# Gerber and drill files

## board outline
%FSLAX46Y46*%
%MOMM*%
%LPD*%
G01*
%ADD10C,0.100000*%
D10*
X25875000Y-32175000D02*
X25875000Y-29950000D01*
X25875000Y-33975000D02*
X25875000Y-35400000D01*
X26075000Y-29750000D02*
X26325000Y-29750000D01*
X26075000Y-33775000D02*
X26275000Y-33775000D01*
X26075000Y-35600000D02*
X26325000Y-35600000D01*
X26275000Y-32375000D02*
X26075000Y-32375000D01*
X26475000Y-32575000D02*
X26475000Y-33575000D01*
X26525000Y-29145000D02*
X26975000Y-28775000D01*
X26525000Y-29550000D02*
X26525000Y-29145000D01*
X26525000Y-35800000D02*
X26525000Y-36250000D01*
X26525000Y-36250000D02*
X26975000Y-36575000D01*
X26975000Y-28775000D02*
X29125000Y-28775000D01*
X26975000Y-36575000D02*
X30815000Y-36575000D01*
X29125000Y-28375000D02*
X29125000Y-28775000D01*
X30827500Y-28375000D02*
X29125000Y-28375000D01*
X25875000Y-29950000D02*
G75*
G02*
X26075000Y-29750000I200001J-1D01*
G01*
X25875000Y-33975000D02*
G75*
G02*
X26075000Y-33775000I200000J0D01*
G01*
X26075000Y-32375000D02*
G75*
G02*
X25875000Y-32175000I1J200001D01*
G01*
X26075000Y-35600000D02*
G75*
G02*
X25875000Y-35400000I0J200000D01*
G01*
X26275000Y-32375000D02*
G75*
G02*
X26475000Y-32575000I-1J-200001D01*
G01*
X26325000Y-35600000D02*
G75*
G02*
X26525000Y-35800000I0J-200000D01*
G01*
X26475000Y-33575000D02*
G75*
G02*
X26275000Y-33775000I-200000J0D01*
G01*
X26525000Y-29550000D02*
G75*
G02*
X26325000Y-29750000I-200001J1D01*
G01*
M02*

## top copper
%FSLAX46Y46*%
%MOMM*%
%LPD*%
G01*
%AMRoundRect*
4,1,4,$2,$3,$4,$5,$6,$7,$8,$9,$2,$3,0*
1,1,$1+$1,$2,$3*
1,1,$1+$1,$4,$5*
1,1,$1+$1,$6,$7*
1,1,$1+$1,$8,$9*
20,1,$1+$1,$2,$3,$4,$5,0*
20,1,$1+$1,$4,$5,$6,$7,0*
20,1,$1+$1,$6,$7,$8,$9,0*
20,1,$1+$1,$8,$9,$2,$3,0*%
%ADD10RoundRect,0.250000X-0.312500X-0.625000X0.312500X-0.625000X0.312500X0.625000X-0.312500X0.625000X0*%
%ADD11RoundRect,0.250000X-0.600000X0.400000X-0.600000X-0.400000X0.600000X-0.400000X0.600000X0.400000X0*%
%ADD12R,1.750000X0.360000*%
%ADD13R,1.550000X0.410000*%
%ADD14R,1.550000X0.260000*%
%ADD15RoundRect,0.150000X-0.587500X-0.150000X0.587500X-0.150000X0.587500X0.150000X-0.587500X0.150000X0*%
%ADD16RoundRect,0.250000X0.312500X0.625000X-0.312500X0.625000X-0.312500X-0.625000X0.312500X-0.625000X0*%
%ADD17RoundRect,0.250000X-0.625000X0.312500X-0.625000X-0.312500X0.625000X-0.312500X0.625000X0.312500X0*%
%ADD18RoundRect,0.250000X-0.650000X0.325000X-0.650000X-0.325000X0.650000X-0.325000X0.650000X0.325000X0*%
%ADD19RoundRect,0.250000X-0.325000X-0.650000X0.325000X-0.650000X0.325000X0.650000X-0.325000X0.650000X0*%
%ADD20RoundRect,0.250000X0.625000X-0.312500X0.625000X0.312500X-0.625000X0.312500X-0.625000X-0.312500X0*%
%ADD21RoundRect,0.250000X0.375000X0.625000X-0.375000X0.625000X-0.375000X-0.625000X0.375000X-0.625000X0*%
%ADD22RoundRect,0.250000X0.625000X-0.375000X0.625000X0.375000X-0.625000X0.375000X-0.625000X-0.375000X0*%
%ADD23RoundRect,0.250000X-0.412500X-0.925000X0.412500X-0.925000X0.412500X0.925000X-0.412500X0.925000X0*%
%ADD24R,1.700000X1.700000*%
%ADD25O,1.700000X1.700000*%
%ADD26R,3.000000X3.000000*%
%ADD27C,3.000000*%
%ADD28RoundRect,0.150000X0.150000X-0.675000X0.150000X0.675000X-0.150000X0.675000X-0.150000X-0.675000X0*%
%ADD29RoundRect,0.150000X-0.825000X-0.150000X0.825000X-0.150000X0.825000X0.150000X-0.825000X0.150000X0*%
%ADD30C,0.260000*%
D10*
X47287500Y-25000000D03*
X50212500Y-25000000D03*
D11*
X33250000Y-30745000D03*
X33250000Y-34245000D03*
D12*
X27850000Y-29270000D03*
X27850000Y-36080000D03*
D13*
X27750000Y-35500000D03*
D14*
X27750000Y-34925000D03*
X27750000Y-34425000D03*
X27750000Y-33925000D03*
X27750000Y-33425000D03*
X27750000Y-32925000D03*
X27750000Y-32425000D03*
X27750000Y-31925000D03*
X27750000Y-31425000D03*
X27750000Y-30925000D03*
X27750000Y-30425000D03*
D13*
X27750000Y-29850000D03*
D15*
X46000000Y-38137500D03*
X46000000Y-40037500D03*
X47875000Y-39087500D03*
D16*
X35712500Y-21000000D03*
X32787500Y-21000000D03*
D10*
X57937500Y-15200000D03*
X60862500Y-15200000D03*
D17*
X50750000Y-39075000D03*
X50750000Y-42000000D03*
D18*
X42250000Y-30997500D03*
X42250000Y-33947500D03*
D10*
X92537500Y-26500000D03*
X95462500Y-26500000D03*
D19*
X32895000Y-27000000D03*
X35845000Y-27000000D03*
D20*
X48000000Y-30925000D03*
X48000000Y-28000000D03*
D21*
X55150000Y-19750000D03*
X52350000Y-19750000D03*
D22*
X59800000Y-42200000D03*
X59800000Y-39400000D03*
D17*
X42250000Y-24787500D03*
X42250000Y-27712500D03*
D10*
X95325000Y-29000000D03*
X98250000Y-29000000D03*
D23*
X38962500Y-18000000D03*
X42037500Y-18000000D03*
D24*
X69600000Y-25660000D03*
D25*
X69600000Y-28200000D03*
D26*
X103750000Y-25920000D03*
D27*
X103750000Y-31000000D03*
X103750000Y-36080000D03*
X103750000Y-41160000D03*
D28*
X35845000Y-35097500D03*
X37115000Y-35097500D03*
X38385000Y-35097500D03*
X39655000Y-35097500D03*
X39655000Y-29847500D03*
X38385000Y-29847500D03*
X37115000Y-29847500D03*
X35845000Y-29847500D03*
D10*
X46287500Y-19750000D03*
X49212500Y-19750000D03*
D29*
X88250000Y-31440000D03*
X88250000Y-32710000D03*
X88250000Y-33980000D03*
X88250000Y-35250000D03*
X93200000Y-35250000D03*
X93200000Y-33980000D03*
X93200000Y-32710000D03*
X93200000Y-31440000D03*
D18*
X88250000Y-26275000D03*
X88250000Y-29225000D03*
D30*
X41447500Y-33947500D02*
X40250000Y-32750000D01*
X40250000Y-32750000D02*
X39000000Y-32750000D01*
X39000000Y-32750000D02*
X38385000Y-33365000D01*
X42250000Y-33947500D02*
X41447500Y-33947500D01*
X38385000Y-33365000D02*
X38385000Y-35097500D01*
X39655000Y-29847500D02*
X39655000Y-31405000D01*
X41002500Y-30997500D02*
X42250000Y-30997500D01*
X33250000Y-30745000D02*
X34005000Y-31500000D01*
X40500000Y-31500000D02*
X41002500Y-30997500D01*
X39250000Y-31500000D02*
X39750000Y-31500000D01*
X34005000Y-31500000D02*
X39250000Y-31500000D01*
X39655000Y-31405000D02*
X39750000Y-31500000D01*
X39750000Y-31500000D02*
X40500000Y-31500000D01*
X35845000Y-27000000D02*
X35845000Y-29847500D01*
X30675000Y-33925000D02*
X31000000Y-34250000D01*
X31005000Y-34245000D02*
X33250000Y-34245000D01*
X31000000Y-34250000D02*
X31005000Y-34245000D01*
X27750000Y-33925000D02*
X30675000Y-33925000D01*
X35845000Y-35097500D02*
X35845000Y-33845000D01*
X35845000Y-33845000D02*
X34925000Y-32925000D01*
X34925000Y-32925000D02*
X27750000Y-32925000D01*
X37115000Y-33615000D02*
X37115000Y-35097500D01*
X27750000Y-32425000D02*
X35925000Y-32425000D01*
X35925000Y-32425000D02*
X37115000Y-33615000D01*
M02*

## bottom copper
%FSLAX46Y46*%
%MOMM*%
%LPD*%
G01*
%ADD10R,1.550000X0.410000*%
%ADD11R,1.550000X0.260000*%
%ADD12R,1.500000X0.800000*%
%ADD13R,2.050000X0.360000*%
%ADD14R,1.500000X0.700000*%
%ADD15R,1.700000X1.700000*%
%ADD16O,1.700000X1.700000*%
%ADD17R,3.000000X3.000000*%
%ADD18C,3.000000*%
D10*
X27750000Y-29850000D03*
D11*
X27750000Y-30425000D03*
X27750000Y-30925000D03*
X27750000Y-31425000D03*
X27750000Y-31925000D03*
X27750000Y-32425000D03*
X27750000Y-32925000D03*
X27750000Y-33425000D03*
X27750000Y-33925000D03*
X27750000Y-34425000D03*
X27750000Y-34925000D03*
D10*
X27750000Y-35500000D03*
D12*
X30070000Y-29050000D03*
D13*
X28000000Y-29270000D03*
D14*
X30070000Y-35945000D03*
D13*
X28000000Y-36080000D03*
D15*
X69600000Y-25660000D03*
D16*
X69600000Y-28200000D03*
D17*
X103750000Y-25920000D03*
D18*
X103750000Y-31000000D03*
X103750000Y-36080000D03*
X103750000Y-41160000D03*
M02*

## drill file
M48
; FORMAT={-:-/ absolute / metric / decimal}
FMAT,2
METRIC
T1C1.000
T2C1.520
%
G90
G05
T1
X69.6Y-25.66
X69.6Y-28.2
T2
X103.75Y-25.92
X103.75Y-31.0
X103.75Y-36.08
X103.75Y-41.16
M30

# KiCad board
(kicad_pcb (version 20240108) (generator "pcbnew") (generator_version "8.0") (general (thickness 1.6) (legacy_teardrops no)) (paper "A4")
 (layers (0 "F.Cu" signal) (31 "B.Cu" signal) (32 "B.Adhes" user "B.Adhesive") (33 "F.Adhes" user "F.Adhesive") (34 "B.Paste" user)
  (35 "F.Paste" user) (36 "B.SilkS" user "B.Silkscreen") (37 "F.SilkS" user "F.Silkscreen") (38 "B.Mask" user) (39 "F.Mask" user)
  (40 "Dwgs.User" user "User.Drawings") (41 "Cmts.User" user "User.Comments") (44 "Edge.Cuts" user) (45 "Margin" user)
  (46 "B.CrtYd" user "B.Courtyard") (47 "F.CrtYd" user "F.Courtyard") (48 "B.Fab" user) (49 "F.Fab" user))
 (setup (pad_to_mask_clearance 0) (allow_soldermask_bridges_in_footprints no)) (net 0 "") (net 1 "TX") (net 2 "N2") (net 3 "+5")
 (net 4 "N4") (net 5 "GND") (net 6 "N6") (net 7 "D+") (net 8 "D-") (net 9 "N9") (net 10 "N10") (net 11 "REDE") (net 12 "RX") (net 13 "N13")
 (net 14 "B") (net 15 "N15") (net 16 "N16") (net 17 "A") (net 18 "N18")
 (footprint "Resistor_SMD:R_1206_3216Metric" (layer "F.Cu") (at 48.75 25)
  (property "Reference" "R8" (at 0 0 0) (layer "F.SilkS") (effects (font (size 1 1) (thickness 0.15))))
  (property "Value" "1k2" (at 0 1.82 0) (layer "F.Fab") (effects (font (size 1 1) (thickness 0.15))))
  (pad "1" smd roundrect (at -1.4625 0) (size 1.125 1.75) (layers "F.Cu" "F.Paste" "F.Mask") (roundrect_rratio 0.222222) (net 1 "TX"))
  (pad "2" smd roundrect (at 1.4625 0) (size 1.125 1.75) (layers "F.Cu" "F.Paste" "F.Mask") (roundrect_rratio 0.222222) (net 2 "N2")))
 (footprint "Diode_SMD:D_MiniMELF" (layer "F.Cu") (at 33.25 32.495 -90)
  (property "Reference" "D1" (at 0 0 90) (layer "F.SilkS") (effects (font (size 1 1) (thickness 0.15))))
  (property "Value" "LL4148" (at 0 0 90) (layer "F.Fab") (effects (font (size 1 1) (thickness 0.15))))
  (pad "1" smd roundrect (at -1.75 0 270) (size 1.3 1.7) (layers "F.Cu" "F.Paste" "F.Mask") (roundrect_rratio 0.1923076923) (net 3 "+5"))
  (pad "2" smd roundrect (at 1.75 0 270) (size 1.3 1.7) (layers "F.Cu" "F.Paste" "F.Mask") (roundrect_rratio 0.1923076923) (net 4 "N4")))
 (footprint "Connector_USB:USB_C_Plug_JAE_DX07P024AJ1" (layer "F.Cu") (at 28.8975 32.675 -90)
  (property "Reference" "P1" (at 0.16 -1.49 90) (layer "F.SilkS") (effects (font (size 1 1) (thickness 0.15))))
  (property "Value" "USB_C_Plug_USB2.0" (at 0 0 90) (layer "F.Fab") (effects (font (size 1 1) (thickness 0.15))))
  (fp_line (start -0.5 3.0225) (end -2.725 3.0225) (stroke (width 0.1) (type solid)) (layer "Edge.Cuts"))
  (fp_line (start 1.3 3.0225) (end 2.725 3.0225) (stroke (width 0.1) (type solid)) (layer "Edge.Cuts"))
  (fp_line (start -2.925 2.8225) (end -2.925 2.5725) (stroke (width 0.1) (type solid)) (layer "Edge.Cuts"))
  (fp_line (start 1.1 2.8225) (end 1.1 2.6225) (stroke (width 0.1) (type solid)) (layer "Edge.Cuts"))
  (fp_line (start 2.925 2.8225) (end 2.925 2.5725) (stroke (width 0.1) (type solid)) (layer "Edge.Cuts"))
  (fp_line (start -0.3 2.6225) (end -0.3 2.8225) (stroke (width 0.1) (type solid)) (layer "Edge.Cuts"))
  (fp_line (start -0.1 2.4225) (end 0.9 2.4225) (stroke (width 0.1) (type solid)) (layer "Edge.Cuts"))
  (fp_line (start -3.53 2.3725) (end -3.9 1.9225) (stroke (width 0.1) (type solid)) (layer "Edge.Cuts"))
  (fp_line (start -3.125 2.3725) (end -3.53 2.3725) (stroke (width 0.1) (type solid)) (layer "Edge.Cuts"))
  (fp_line (start 3.125 2.3725) (end 3.575 2.3725) (stroke (width 0.1) (type solid)) (layer "Edge.Cuts"))
  (fp_line (start 3.575 2.3725) (end 3.9 1.9225) (stroke (width 0.1) (type solid)) (layer "Edge.Cuts"))
  (fp_line (start -3.9 1.9225) (end -3.9 -0.2275) (stroke (width 0.1) (type solid)) (layer "Edge.Cuts"))
  (fp_line (start 3.9 1.9225) (end 3.9 -1.9175) (stroke (width 0.1) (type solid)) (layer "Edge.Cuts"))
  (fp_line (start -4.3 -0.2275) (end -3.9 -0.2275) (stroke (width 0.1) (type solid)) (layer "Edge.Cuts"))
  (fp_line (start -4.3 -1.93) (end -4.3 -0.2275) (stroke (width 0.1) (type solid)) (layer "Edge.Cuts"))
  (fp_arc (start -2.725 3.0225) (mid -2.866421 2.963921) (end -2.925 2.8225) (stroke (width 0.1) (type solid)) (layer "Edge.Cuts"))
  (fp_arc (start 1.3 3.0225) (mid 1.158579 2.963921) (end 1.1 2.8225) (stroke (width 0.1) (type solid)) (layer "Edge.Cuts"))
  (fp_arc (start -0.3 2.8225) (mid -0.358579 2.963921) (end -0.5 3.0225) (stroke (width 0.1) (type solid)) (layer "Edge.Cuts"))
  (fp_arc (start 2.925 2.8225) (mid 2.866421 2.963921) (end 2.725 3.0225) (stroke (width 0.1) (type solid)) (layer "Edge.Cuts"))
  (fp_arc (start -0.3 2.6225) (mid -0.241421 2.481079) (end -0.1 2.4225) (stroke (width 0.1) (type solid)) (layer "Edge.Cuts"))
  (fp_arc (start 2.925 2.5725) (mid 2.983579 2.431079) (end 3.125 2.3725) (stroke (width 0.1) (type solid)) (layer "Edge.Cuts"))
  (fp_arc (start 0.9 2.4225) (mid 1.041421 2.481079) (end 1.1 2.6225) (stroke (width 0.1) (type solid)) (layer "Edge.Cuts"))
  (fp_arc (start -3.125 2.3725) (mid -2.983579 2.431079) (end -2.925 2.5725) (stroke (width 0.1) (type solid)) (layer "Edge.Cuts"))
  (pad "" smd rect (at -3.405 1.0475 270) (size 0.36 1.75) (layers "F.Cu" "F.Mask"))
  (pad "" smd rect (at 3.405 1.0475 270) (size 0.36 1.75) (layers "F.Cu" "F.Mask"))
  (pad "A1" smd rect (at 2.825 1.1475 270) (size 0.41 1.55) (layers "F.Cu" "F.Paste" "F.Mask") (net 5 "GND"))
  (pad "A2" smd rect (at 2.25 1.1475 270) (size 0.26 1.55) (layers "F.Cu" "F.Paste" "F.Mask"))
  (pad "A3" smd rect (at 1.75 1.1475 270) (size 0.26 1.55) (layers "F.Cu" "F.Paste" "F.Mask"))
  (pad "A4" smd rect (at 1.25 1.1475 270) (size 0.26 1.55) (layers "F.Cu" "F.Paste" "F.Mask") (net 4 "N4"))
  (pad "A5" smd rect (at 0.75 1.1475 270) (size 0.26 1.55) (layers "F.Cu" "F.Paste" "F.Mask") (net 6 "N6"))
  (pad "A6" smd rect (at 0.25 1.1475 90) (size 0.26 1.55) (layers "F.Cu" "F.Paste" "F.Mask") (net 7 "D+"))
  (pad "A7" smd rect (at -0.25 1.1475 90) (size 0.26 1.55) (layers "F.Cu" "F.Paste" "F.Mask") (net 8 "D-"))
  (pad "A8" smd rect (at -0.75 1.1475 270) (size 0.26 1.55) (layers "F.Cu" "F.Paste" "F.Mask"))
  (pad "A9" smd rect (at -1.25 1.1475 270) (size 0.26 1.55) (layers "F.Cu" "F.Paste" "F.Mask") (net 4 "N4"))
  (pad "A10" smd rect (at -1.75 1.1475 270) (size 0.26 1.55) (layers "F.Cu" "F.Paste" "F.Mask"))
  (pad "A11" smd rect (at -2.25 1.1475 270) (size 0.26 1.55) (layers "F.Cu" "F.Paste" "F.Mask"))
  (pad "A12" smd rect (at -2.825 1.1475 270) (size 0.41 1.55) (layers "F.Cu" "F.Paste" "F.Mask") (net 5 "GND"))
  (pad "B1" smd rect (at -2.825 1.1475 270) (size 0.41 1.55) (layers "B.Cu" "B.Paste" "B.Mask") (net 5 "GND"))
  (pad "B2" smd rect (at -2.25 1.1475 270) (size 0.26 1.55) (layers "B.Cu" "B.Paste" "B.Mask"))
  (pad "B3" smd rect (at -1.75 1.1475 270) (size 0.26 1.55) (layers "B.Cu" "B.Paste" "B.Mask"))
  (pad "B4" smd rect (at -1.25 1.1475 270) (size 0.26 1.55) (layers "B.Cu" "B.Paste" "B.Mask") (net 4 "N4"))
  (pad "B5" smd rect (at -0.75 1.1475 270) (size 0.26 1.55) (layers "B.Cu" "B.Paste" "B.Mask") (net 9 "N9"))
  (pad "B6" smd rect (at -0.25 1.1475 90) (size 0.26 1.55) (layers "B.Cu" "B.Paste" "B.Mask"))
  (pad "B7" smd rect (at 0.25 1.1475 270) (size 0.26 1.55) (layers "B.Cu" "B.Paste" "B.Mask"))
  (pad "B8" smd rect (at 0.75 1.1475 270) (size 0.26 1.55) (layers "B.Cu" "B.Paste" "B.Mask"))
  (pad "B9" smd rect (at 1.25 1.1475 270) (size 0.26 1.55) (layers "B.Cu" "B.Paste" "B.Mask") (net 4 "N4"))
  (pad "B10" smd rect (at 1.75 1.1475 270) (size 0.26 1.55) (layers "B.Cu" "B.Paste" "B.Mask"))
  (pad "B11" smd rect (at 2.25 1.1475 270) (size 0.26 1.55) (layers "B.Cu" "B.Paste" "B.Mask"))
  (pad "B12" smd rect (at 2.825 1.1475 270) (size 0.41 1.55) (layers "B.Cu" "B.Paste" "B.Mask") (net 5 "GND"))
  (pad "S1" smd rect (at -3.625 -1.1725 270) (size 0.8 1.5) (layers "B.Cu" "B.Paste" "B.Mask") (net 5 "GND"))
  (pad "S1" smd rect (at -3.405 0.8975 270) (size 0.36 2.05) (layers "B.Cu" "B.Paste" "B.Mask") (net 5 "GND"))
  (pad "S1" smd rect (at 3.27 -1.1725 90) (size 0.7 1.5) (layers "B.Cu" "B.Paste" "B.Mask") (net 5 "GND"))
  (pad "S1" smd rect (at 3.405 0.8975 270) (size 0.36 2.05) (layers "B.Cu" "B.Paste" "B.Mask") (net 5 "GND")))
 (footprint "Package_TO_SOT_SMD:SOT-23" (layer "F.Cu") (at 46.9375 39.0875)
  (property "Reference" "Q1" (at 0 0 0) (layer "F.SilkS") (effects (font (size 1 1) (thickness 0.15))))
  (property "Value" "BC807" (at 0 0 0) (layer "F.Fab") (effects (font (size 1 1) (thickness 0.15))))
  (pad "1" smd roundrect (at -0.9375 -0.95) (size 1.475 0.6) (layers "F.Cu" "F.Paste" "F.Mask") (roundrect_rratio 0.25) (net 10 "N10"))
  (pad "2" smd roundrect (at -0.9375 0.95) (size 1.475 0.6) (layers "F.Cu" "F.Paste" "F.Mask") (roundrect_rratio 0.25) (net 3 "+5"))
  (pad "3" smd roundrect (at 0.9375 0) (size 1.475 0.6) (layers "F.Cu" "F.Paste" "F.Mask") (roundrect_rratio 0.25) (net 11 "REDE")))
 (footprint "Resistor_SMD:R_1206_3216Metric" (layer "F.Cu") (at 34.25 21 180)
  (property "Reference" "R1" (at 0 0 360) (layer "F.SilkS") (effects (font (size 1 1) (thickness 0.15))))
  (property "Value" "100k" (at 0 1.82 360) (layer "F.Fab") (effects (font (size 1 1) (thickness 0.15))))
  (pad "1" smd roundrect (at -1.4625 0 180) (size 1.125 1.75) (layers "F.Cu" "F.Paste" "F.Mask") (roundrect_rratio 0.222222) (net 3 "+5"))
  (pad "2" smd roundrect (at 1.4625 0 180) (size 1.125 1.75) (layers "F.Cu" "F.Paste" "F.Mask") (roundrect_rratio 0.222222) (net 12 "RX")))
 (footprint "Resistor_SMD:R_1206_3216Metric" (layer "F.Cu") (at 59.4 15.2)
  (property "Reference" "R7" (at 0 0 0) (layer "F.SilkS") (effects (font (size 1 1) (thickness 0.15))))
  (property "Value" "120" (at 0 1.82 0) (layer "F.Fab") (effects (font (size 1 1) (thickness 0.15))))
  (pad "1" smd roundrect (at -1.4625 0) (size 1.125 1.75) (layers "F.Cu" "F.Paste" "F.Mask") (roundrect_rratio 0.222222) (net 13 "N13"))
  (pad "2" smd roundrect (at 1.4625 0) (size 1.125 1.75) (layers "F.Cu" "F.Paste" "F.Mask") (roundrect_rratio 0.222222) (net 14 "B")))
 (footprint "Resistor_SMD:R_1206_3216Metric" (layer "F.Cu") (at 50.75 40.5375 -90)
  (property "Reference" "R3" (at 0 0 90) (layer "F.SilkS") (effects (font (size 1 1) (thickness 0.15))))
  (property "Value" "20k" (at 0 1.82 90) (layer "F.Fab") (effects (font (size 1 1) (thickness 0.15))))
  (pad "1" smd roundrect (at -1.4625 0 270) (size 1.125 1.75) (layers "F.Cu" "F.Paste" "F.Mask") (roundrect_rratio 0.222222) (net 11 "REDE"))
  (pad "2" smd roundrect (at 1.4625 0 270) (size 1.125 1.75) (layers "F.Cu" "F.Paste" "F.Mask") (roundrect_rratio 0.222222) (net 5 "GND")))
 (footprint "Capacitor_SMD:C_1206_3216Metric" (layer "F.Cu") (at 42.25 32.4725 -90)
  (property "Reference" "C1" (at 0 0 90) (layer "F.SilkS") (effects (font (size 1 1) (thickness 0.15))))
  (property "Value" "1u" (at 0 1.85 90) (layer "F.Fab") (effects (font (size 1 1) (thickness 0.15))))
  (pad "1" smd roundrect (at -1.475 0 270) (size 1.15 1.8) (layers "F.Cu" "F.Paste" "F.Mask") (roundrect_rratio 0.217391) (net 3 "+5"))
  (pad "2" smd roundrect (at 1.475 0 270) (size 1.15 1.8) (layers "F.Cu" "F.Paste" "F.Mask") (roundrect_rratio 0.217391) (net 5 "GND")))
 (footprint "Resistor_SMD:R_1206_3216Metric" (layer "F.Cu") (at 94 26.5)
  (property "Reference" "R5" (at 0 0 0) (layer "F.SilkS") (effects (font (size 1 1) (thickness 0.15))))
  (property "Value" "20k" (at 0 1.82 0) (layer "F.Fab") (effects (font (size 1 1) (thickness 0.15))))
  (pad "1" smd roundrect (at -1.4625 0) (size 1.125 1.75) (layers "F.Cu" "F.Paste" "F.Mask") (roundrect_rratio 0.222222) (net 14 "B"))
  (pad "2" smd roundrect (at 1.4625 0) (size 1.125 1.75) (layers "F.Cu" "F.Paste" "F.Mask") (roundrect_rratio 0.222222) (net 5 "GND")))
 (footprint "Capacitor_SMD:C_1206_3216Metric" (layer "F.Cu") (at 34.37 27)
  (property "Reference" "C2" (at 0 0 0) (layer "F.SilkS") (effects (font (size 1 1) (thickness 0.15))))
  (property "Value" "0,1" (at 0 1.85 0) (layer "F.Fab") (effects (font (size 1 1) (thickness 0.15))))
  (pad "1" smd roundrect (at -1.475 0) (size 1.15 1.8) (layers "F.Cu" "F.Paste" "F.Mask") (roundrect_rratio 0.217391) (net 5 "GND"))
  (pad "2" smd roundrect (at 1.475 0) (size 1.15 1.8) (layers "F.Cu" "F.Paste" "F.Mask") (roundrect_rratio 0.217391) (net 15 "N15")))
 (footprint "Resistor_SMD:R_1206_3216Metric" (layer "F.Cu") (at 48 29.4625 90)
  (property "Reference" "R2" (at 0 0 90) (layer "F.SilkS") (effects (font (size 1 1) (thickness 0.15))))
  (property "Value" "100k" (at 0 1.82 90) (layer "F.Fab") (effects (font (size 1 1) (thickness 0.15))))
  (pad "1" smd roundrect (at -1.4625 0 90) (size 1.125 1.75) (layers "F.Cu" "F.Paste" "F.Mask") (roundrect_rratio 0.222222) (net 3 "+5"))
  (pad "2" smd roundrect (at 1.4625 0 90) (size 1.125 1.75) (layers "F.Cu" "F.Paste" "F.Mask") (roundrect_rratio 0.222222) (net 1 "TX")))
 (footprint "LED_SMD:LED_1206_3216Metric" (layer "F.Cu") (at 53.75 19.75 180)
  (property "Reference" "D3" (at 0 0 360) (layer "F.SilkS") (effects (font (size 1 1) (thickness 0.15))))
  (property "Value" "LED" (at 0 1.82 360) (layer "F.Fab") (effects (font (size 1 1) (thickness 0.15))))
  (pad "1" smd roundrect (at -1.4 0 180) (size 1.25 1.75) (layers "F.Cu" "F.Paste" "F.Mask") (roundrect_rratio 0.2) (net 5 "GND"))
  (pad "2" smd roundrect (at 1.4 0 180) (size 1.25 1.75) (layers "F.Cu" "F.Paste" "F.Mask") (roundrect_rratio 0.2) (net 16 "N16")))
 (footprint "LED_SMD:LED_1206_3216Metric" (layer "F.Cu") (at 59.8 40.8 90)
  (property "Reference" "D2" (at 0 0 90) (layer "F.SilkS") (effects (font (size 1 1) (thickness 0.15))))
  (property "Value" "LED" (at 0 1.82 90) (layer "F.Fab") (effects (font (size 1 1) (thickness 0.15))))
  (pad "1" smd roundrect (at -1.4 0 90) (size 1.25 1.75) (layers "F.Cu" "F.Paste" "F.Mask") (roundrect_rratio 0.2) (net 5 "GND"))
  (pad "2" smd roundrect (at 1.4 0 90) (size 1.25 1.75) (layers "F.Cu" "F.Paste" "F.Mask") (roundrect_rratio 0.2) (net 2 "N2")))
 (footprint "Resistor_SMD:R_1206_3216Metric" (layer "F.Cu") (at 42.25 26.25 -90)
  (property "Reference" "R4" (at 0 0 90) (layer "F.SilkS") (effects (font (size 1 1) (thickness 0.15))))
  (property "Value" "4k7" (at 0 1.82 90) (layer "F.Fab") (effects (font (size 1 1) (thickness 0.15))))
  (pad "1" smd roundrect (at -1.4625 0 270) (size 1.125 1.75) (layers "F.Cu" "F.Paste" "F.Mask") (roundrect_rratio 0.222222) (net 1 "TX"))
  (pad "2" smd roundrect (at 1.4625 0 270) (size 1.125 1.75) (layers "F.Cu" "F.Paste" "F.Mask") (roundrect_rratio 0.222222) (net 10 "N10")))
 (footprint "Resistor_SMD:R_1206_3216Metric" (layer "F.Cu") (at 96.7875 29)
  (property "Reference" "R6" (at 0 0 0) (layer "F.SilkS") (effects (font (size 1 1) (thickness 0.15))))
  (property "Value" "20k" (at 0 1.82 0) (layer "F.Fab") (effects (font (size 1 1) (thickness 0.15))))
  (pad "1" smd roundrect (at -1.4625 0) (size 1.125 1.75) (layers "F.Cu" "F.Paste" "F.Mask") (roundrect_rratio 0.222222) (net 3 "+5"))
  (pad "2" smd roundrect (at 1.4625 0) (size 1.125 1.75) (layers "F.Cu" "F.Paste" "F.Mask") (roundrect_rratio 0.222222) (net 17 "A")))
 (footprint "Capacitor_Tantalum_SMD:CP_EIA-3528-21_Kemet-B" (layer "F.Cu") (at 40.5 18)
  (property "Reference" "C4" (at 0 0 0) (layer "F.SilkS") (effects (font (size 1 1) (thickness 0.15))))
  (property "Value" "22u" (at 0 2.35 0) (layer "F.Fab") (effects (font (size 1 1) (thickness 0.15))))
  (pad "1" smd roundrect (at -1.5375 0) (size 1.325 2.35) (layers "F.Cu" "F.Paste" "F.Mask") (roundrect_rratio 0.188679) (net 3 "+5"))
  (pad "2" smd roundrect (at 1.5375 0) (size 1.325 2.35) (layers "F.Cu" "F.Paste" "F.Mask") (roundrect_rratio 0.188679) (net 5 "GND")))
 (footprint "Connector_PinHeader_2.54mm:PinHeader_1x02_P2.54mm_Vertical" (layer "F.Cu") (at 69.6 25.66)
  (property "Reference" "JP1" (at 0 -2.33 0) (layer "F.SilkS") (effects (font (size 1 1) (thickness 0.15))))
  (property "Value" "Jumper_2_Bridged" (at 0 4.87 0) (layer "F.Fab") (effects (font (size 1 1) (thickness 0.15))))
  (pad "1" thru_hole rect (at 0 0) (size 1.7 1.7) (drill 1) (layers "*.Cu" "*.Mask") (remove_unused_layers no) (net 13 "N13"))
  (pad "2" thru_hole oval (at 0 2.54) (size 1.7 1.7) (drill 1) (layers "*.Cu" "*.Mask") (remove_unused_layers no) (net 17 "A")))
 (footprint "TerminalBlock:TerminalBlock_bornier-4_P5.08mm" (layer "F.Cu") (at 103.75 25.92 -90)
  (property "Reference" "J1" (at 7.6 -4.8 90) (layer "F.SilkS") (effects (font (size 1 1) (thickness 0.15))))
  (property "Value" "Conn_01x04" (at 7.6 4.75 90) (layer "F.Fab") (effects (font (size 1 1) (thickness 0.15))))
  (pad "1" thru_hole rect (at 0 0 270) (size 3 3) (drill 1.52) (layers "*.Cu" "*.Mask") (remove_unused_layers no) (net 3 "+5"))
  (pad "2" thru_hole circle (at 5.08 0 270) (size 3 3) (drill 1.52) (layers "*.Cu" "*.Mask") (remove_unused_layers no) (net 14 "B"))
  (pad "3" thru_hole circle (at 10.16 0 270) (size 3 3) (drill 1.52) (layers "*.Cu" "*.Mask") (remove_unused_layers no) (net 17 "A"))
  (pad "4" thru_hole circle (at 15.24 0 270) (size 3 3) (drill 1.52) (layers "*.Cu" "*.Mask") (remove_unused_layers no) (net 5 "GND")))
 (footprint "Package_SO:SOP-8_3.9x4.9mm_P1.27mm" (layer "F.Cu") (at 37.75 32.4725 90)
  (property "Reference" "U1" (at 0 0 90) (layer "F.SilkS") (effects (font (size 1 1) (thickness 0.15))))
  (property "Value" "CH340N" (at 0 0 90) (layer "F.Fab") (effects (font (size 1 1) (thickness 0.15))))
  (pad "1" smd roundrect (at -2.625 -1.905 90) (size 1.65 0.6) (layers "F.Cu" "F.Paste" "F.Mask") (roundrect_rratio 0.25) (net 7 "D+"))
  (pad "2" smd roundrect (at -2.625 -0.635 90) (size 1.65 0.6) (layers "F.Cu" "F.Paste" "F.Mask") (roundrect_rratio 0.25) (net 8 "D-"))
  (pad "3" smd roundrect (at -2.625 0.635 90) (size 1.65 0.6) (layers "F.Cu" "F.Paste" "F.Mask") (roundrect_rratio 0.25) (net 5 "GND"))
  (pad "4" smd roundrect (at -2.625 1.905 90) (size 1.65 0.6) (layers "F.Cu" "F.Paste" "F.Mask") (roundrect_rratio 0.25) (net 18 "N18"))
  (pad "5" smd roundrect (at 2.625 1.905 90) (size 1.65 0.6) (layers "F.Cu" "F.Paste" "F.Mask") (roundrect_rratio 0.25) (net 3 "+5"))
  (pad "6" smd roundrect (at 2.625 0.635 90) (size 1.65 0.6) (layers "F.Cu" "F.Paste" "F.Mask") (roundrect_rratio 0.25) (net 1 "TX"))
  (pad "7" smd roundrect (at 2.625 -0.635 90) (size 1.65 0.6) (layers "F.Cu" "F.Paste" "F.Mask") (roundrect_rratio 0.25) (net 12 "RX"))
  (pad "8" smd roundrect (at 2.625 -1.905 90) (size 1.65 0.6) (layers "F.Cu" "F.Paste" "F.Mask") (roundrect_rratio 0.25) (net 15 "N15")))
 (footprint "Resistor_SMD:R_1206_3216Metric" (layer "F.Cu") (at 47.75 19.75)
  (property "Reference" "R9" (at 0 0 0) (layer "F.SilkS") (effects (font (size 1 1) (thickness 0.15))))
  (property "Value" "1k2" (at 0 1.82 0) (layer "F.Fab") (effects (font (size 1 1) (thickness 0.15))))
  (pad "1" smd roundrect (at -1.4625 0) (size 1.125 1.75) (layers "F.Cu" "F.Paste" "F.Mask") (roundrect_rratio 0.222222) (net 12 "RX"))
  (pad "2" smd roundrect (at 1.4625 0) (size 1.125 1.75) (layers "F.Cu" "F.Paste" "F.Mask") (roundrect_rratio 0.222222) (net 16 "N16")))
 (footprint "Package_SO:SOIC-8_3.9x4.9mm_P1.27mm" (layer "F.Cu") (at 90.725 33.345)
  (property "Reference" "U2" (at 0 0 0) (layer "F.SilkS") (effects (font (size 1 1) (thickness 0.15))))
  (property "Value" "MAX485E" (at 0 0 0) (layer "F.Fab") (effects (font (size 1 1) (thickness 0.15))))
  (pad "1" smd roundrect (at -2.475 -1.905) (size 1.95 0.6) (layers "F.Cu" "F.Paste" "F.Mask") (roundrect_rratio 0.25) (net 12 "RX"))
  (pad "2" smd roundrect (at -2.475 -0.635) (size 1.95 0.6) (layers "F.Cu" "F.Paste" "F.Mask") (roundrect_rratio 0.25) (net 11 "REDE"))
  (pad "3" smd roundrect (at -2.475 0.635) (size 1.95 0.6) (layers "F.Cu" "F.Paste" "F.Mask") (roundrect_rratio 0.25) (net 11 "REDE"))
  (pad "4" smd roundrect (at -2.475 1.905) (size 1.95 0.6) (layers "F.Cu" "F.Paste" "F.Mask") (roundrect_rratio 0.25) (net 1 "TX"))
  (pad "5" smd roundrect (at 2.475 1.905) (size 1.95 0.6) (layers "F.Cu" "F.Paste" "F.Mask") (roundrect_rratio 0.25) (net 5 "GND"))
  (pad "6" smd roundrect (at 2.475 0.635) (size 1.95 0.6) (layers "F.Cu" "F.Paste" "F.Mask") (roundrect_rratio 0.25) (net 17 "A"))
  (pad "7" smd roundrect (at 2.475 -0.635) (size 1.95 0.6) (layers "F.Cu" "F.Paste" "F.Mask") (roundrect_rratio 0.25) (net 14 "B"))
  (pad "8" smd roundrect (at 2.475 -1.905) (size 1.95 0.6) (layers "F.Cu" "F.Paste" "F.Mask") (roundrect_rratio 0.25) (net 3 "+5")))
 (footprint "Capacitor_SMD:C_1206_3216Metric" (layer "F.Cu") (at 88.25 27.75 -90)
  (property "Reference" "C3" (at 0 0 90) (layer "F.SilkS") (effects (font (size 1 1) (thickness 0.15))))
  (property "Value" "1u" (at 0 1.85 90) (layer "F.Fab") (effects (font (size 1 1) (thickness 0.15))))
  (pad "1" smd roundrect (at -1.475 0 270) (size 1.15 1.8) (layers "F.Cu" "F.Paste" "F.Mask") (roundrect_rratio 0.217391) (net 3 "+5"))
  (pad "2" smd roundrect (at 1.475 0 270) (size 1.15 1.8) (layers "F.Cu" "F.Paste" "F.Mask") (roundrect_rratio 0.217391) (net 5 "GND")))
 (segment (start 41.4475 33.9475) (end 40.25 32.75) (width 0.26) (layer "F.Cu") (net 5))
 (segment (start 40.25 32.75) (end 39 32.75) (width 0.26) (layer "F.Cu") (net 5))
 (segment (start 39 32.75) (end 38.385 33.365) (width 0.26) (layer "F.Cu") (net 5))
 (segment (start 42.25 33.9475) (end 41.4475 33.9475) (width 0.26) (layer "F.Cu") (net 5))
 (segment (start 38.385 33.365) (end 38.385 35.0975) (width 0.26) (layer "F.Cu") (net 5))
 (segment (start 39.655 29.8475) (end 39.655 31.405) (width 0.26) (layer "F.Cu") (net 3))
 (segment (start 41.0025 30.9975) (end 42.25 30.9975) (width 0.26) (layer "F.Cu") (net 3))
 (segment (start 33.25 30.745) (end 34.005 31.5) (width 0.26) (layer "F.Cu") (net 3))
 (segment (start 40.5 31.5) (end 41.0025 30.9975) (width 0.26) (layer "F.Cu") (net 3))
 (segment (start 39.25 31.5) (end 39.75 31.5) (width 0.26) (layer "F.Cu") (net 3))
 (segment (start 34.005 31.5) (end 39.25 31.5) (width 0.26) (layer "F.Cu") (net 3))
 (segment (start 39.655 31.405) (end 39.75 31.5) (width 0.26) (layer "F.Cu") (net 3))
 (segment (start 39.75 31.5) (end 40.5 31.5) (width 0.26) (layer "F.Cu") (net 3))
 (segment (start 35.845 27) (end 35.845 29.8475) (width 0.26) (layer "F.Cu") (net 15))
 (segment (start 30.675 33.925) (end 31 34.25) (width 0.26) (layer "F.Cu") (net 4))
 (segment (start 31.005 34.245) (end 33.25 34.245) (width 0.26) (layer "F.Cu") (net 4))
 (segment (start 31 34.25) (end 31.005 34.245) (width 0.26) (layer "F.Cu") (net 4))
 (segment (start 27.75 33.925) (end 30.675 33.925) (width 0.26) (layer "F.Cu") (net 4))
 (segment (start 35.845 35.0975) (end 35.845 33.845) (width 0.26) (layer "F.Cu") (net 7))
 (segment (start 35.845 33.845) (end 34.925 32.925) (width 0.26) (layer "F.Cu") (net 7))
 (segment (start 34.925 32.925) (end 27.75 32.925) (width 0.26) (layer "F.Cu") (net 7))
 (segment (start 37.115 33.615) (end 37.115 35.0975) (width 0.26) (layer "F.Cu") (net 8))
 (segment (start 27.75 32.425) (end 35.925 32.425) (width 0.26) (layer "F.Cu") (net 8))
 (segment (start 35.925 32.425) (end 37.115 33.615) (width 0.26) (layer "F.Cu") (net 8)))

